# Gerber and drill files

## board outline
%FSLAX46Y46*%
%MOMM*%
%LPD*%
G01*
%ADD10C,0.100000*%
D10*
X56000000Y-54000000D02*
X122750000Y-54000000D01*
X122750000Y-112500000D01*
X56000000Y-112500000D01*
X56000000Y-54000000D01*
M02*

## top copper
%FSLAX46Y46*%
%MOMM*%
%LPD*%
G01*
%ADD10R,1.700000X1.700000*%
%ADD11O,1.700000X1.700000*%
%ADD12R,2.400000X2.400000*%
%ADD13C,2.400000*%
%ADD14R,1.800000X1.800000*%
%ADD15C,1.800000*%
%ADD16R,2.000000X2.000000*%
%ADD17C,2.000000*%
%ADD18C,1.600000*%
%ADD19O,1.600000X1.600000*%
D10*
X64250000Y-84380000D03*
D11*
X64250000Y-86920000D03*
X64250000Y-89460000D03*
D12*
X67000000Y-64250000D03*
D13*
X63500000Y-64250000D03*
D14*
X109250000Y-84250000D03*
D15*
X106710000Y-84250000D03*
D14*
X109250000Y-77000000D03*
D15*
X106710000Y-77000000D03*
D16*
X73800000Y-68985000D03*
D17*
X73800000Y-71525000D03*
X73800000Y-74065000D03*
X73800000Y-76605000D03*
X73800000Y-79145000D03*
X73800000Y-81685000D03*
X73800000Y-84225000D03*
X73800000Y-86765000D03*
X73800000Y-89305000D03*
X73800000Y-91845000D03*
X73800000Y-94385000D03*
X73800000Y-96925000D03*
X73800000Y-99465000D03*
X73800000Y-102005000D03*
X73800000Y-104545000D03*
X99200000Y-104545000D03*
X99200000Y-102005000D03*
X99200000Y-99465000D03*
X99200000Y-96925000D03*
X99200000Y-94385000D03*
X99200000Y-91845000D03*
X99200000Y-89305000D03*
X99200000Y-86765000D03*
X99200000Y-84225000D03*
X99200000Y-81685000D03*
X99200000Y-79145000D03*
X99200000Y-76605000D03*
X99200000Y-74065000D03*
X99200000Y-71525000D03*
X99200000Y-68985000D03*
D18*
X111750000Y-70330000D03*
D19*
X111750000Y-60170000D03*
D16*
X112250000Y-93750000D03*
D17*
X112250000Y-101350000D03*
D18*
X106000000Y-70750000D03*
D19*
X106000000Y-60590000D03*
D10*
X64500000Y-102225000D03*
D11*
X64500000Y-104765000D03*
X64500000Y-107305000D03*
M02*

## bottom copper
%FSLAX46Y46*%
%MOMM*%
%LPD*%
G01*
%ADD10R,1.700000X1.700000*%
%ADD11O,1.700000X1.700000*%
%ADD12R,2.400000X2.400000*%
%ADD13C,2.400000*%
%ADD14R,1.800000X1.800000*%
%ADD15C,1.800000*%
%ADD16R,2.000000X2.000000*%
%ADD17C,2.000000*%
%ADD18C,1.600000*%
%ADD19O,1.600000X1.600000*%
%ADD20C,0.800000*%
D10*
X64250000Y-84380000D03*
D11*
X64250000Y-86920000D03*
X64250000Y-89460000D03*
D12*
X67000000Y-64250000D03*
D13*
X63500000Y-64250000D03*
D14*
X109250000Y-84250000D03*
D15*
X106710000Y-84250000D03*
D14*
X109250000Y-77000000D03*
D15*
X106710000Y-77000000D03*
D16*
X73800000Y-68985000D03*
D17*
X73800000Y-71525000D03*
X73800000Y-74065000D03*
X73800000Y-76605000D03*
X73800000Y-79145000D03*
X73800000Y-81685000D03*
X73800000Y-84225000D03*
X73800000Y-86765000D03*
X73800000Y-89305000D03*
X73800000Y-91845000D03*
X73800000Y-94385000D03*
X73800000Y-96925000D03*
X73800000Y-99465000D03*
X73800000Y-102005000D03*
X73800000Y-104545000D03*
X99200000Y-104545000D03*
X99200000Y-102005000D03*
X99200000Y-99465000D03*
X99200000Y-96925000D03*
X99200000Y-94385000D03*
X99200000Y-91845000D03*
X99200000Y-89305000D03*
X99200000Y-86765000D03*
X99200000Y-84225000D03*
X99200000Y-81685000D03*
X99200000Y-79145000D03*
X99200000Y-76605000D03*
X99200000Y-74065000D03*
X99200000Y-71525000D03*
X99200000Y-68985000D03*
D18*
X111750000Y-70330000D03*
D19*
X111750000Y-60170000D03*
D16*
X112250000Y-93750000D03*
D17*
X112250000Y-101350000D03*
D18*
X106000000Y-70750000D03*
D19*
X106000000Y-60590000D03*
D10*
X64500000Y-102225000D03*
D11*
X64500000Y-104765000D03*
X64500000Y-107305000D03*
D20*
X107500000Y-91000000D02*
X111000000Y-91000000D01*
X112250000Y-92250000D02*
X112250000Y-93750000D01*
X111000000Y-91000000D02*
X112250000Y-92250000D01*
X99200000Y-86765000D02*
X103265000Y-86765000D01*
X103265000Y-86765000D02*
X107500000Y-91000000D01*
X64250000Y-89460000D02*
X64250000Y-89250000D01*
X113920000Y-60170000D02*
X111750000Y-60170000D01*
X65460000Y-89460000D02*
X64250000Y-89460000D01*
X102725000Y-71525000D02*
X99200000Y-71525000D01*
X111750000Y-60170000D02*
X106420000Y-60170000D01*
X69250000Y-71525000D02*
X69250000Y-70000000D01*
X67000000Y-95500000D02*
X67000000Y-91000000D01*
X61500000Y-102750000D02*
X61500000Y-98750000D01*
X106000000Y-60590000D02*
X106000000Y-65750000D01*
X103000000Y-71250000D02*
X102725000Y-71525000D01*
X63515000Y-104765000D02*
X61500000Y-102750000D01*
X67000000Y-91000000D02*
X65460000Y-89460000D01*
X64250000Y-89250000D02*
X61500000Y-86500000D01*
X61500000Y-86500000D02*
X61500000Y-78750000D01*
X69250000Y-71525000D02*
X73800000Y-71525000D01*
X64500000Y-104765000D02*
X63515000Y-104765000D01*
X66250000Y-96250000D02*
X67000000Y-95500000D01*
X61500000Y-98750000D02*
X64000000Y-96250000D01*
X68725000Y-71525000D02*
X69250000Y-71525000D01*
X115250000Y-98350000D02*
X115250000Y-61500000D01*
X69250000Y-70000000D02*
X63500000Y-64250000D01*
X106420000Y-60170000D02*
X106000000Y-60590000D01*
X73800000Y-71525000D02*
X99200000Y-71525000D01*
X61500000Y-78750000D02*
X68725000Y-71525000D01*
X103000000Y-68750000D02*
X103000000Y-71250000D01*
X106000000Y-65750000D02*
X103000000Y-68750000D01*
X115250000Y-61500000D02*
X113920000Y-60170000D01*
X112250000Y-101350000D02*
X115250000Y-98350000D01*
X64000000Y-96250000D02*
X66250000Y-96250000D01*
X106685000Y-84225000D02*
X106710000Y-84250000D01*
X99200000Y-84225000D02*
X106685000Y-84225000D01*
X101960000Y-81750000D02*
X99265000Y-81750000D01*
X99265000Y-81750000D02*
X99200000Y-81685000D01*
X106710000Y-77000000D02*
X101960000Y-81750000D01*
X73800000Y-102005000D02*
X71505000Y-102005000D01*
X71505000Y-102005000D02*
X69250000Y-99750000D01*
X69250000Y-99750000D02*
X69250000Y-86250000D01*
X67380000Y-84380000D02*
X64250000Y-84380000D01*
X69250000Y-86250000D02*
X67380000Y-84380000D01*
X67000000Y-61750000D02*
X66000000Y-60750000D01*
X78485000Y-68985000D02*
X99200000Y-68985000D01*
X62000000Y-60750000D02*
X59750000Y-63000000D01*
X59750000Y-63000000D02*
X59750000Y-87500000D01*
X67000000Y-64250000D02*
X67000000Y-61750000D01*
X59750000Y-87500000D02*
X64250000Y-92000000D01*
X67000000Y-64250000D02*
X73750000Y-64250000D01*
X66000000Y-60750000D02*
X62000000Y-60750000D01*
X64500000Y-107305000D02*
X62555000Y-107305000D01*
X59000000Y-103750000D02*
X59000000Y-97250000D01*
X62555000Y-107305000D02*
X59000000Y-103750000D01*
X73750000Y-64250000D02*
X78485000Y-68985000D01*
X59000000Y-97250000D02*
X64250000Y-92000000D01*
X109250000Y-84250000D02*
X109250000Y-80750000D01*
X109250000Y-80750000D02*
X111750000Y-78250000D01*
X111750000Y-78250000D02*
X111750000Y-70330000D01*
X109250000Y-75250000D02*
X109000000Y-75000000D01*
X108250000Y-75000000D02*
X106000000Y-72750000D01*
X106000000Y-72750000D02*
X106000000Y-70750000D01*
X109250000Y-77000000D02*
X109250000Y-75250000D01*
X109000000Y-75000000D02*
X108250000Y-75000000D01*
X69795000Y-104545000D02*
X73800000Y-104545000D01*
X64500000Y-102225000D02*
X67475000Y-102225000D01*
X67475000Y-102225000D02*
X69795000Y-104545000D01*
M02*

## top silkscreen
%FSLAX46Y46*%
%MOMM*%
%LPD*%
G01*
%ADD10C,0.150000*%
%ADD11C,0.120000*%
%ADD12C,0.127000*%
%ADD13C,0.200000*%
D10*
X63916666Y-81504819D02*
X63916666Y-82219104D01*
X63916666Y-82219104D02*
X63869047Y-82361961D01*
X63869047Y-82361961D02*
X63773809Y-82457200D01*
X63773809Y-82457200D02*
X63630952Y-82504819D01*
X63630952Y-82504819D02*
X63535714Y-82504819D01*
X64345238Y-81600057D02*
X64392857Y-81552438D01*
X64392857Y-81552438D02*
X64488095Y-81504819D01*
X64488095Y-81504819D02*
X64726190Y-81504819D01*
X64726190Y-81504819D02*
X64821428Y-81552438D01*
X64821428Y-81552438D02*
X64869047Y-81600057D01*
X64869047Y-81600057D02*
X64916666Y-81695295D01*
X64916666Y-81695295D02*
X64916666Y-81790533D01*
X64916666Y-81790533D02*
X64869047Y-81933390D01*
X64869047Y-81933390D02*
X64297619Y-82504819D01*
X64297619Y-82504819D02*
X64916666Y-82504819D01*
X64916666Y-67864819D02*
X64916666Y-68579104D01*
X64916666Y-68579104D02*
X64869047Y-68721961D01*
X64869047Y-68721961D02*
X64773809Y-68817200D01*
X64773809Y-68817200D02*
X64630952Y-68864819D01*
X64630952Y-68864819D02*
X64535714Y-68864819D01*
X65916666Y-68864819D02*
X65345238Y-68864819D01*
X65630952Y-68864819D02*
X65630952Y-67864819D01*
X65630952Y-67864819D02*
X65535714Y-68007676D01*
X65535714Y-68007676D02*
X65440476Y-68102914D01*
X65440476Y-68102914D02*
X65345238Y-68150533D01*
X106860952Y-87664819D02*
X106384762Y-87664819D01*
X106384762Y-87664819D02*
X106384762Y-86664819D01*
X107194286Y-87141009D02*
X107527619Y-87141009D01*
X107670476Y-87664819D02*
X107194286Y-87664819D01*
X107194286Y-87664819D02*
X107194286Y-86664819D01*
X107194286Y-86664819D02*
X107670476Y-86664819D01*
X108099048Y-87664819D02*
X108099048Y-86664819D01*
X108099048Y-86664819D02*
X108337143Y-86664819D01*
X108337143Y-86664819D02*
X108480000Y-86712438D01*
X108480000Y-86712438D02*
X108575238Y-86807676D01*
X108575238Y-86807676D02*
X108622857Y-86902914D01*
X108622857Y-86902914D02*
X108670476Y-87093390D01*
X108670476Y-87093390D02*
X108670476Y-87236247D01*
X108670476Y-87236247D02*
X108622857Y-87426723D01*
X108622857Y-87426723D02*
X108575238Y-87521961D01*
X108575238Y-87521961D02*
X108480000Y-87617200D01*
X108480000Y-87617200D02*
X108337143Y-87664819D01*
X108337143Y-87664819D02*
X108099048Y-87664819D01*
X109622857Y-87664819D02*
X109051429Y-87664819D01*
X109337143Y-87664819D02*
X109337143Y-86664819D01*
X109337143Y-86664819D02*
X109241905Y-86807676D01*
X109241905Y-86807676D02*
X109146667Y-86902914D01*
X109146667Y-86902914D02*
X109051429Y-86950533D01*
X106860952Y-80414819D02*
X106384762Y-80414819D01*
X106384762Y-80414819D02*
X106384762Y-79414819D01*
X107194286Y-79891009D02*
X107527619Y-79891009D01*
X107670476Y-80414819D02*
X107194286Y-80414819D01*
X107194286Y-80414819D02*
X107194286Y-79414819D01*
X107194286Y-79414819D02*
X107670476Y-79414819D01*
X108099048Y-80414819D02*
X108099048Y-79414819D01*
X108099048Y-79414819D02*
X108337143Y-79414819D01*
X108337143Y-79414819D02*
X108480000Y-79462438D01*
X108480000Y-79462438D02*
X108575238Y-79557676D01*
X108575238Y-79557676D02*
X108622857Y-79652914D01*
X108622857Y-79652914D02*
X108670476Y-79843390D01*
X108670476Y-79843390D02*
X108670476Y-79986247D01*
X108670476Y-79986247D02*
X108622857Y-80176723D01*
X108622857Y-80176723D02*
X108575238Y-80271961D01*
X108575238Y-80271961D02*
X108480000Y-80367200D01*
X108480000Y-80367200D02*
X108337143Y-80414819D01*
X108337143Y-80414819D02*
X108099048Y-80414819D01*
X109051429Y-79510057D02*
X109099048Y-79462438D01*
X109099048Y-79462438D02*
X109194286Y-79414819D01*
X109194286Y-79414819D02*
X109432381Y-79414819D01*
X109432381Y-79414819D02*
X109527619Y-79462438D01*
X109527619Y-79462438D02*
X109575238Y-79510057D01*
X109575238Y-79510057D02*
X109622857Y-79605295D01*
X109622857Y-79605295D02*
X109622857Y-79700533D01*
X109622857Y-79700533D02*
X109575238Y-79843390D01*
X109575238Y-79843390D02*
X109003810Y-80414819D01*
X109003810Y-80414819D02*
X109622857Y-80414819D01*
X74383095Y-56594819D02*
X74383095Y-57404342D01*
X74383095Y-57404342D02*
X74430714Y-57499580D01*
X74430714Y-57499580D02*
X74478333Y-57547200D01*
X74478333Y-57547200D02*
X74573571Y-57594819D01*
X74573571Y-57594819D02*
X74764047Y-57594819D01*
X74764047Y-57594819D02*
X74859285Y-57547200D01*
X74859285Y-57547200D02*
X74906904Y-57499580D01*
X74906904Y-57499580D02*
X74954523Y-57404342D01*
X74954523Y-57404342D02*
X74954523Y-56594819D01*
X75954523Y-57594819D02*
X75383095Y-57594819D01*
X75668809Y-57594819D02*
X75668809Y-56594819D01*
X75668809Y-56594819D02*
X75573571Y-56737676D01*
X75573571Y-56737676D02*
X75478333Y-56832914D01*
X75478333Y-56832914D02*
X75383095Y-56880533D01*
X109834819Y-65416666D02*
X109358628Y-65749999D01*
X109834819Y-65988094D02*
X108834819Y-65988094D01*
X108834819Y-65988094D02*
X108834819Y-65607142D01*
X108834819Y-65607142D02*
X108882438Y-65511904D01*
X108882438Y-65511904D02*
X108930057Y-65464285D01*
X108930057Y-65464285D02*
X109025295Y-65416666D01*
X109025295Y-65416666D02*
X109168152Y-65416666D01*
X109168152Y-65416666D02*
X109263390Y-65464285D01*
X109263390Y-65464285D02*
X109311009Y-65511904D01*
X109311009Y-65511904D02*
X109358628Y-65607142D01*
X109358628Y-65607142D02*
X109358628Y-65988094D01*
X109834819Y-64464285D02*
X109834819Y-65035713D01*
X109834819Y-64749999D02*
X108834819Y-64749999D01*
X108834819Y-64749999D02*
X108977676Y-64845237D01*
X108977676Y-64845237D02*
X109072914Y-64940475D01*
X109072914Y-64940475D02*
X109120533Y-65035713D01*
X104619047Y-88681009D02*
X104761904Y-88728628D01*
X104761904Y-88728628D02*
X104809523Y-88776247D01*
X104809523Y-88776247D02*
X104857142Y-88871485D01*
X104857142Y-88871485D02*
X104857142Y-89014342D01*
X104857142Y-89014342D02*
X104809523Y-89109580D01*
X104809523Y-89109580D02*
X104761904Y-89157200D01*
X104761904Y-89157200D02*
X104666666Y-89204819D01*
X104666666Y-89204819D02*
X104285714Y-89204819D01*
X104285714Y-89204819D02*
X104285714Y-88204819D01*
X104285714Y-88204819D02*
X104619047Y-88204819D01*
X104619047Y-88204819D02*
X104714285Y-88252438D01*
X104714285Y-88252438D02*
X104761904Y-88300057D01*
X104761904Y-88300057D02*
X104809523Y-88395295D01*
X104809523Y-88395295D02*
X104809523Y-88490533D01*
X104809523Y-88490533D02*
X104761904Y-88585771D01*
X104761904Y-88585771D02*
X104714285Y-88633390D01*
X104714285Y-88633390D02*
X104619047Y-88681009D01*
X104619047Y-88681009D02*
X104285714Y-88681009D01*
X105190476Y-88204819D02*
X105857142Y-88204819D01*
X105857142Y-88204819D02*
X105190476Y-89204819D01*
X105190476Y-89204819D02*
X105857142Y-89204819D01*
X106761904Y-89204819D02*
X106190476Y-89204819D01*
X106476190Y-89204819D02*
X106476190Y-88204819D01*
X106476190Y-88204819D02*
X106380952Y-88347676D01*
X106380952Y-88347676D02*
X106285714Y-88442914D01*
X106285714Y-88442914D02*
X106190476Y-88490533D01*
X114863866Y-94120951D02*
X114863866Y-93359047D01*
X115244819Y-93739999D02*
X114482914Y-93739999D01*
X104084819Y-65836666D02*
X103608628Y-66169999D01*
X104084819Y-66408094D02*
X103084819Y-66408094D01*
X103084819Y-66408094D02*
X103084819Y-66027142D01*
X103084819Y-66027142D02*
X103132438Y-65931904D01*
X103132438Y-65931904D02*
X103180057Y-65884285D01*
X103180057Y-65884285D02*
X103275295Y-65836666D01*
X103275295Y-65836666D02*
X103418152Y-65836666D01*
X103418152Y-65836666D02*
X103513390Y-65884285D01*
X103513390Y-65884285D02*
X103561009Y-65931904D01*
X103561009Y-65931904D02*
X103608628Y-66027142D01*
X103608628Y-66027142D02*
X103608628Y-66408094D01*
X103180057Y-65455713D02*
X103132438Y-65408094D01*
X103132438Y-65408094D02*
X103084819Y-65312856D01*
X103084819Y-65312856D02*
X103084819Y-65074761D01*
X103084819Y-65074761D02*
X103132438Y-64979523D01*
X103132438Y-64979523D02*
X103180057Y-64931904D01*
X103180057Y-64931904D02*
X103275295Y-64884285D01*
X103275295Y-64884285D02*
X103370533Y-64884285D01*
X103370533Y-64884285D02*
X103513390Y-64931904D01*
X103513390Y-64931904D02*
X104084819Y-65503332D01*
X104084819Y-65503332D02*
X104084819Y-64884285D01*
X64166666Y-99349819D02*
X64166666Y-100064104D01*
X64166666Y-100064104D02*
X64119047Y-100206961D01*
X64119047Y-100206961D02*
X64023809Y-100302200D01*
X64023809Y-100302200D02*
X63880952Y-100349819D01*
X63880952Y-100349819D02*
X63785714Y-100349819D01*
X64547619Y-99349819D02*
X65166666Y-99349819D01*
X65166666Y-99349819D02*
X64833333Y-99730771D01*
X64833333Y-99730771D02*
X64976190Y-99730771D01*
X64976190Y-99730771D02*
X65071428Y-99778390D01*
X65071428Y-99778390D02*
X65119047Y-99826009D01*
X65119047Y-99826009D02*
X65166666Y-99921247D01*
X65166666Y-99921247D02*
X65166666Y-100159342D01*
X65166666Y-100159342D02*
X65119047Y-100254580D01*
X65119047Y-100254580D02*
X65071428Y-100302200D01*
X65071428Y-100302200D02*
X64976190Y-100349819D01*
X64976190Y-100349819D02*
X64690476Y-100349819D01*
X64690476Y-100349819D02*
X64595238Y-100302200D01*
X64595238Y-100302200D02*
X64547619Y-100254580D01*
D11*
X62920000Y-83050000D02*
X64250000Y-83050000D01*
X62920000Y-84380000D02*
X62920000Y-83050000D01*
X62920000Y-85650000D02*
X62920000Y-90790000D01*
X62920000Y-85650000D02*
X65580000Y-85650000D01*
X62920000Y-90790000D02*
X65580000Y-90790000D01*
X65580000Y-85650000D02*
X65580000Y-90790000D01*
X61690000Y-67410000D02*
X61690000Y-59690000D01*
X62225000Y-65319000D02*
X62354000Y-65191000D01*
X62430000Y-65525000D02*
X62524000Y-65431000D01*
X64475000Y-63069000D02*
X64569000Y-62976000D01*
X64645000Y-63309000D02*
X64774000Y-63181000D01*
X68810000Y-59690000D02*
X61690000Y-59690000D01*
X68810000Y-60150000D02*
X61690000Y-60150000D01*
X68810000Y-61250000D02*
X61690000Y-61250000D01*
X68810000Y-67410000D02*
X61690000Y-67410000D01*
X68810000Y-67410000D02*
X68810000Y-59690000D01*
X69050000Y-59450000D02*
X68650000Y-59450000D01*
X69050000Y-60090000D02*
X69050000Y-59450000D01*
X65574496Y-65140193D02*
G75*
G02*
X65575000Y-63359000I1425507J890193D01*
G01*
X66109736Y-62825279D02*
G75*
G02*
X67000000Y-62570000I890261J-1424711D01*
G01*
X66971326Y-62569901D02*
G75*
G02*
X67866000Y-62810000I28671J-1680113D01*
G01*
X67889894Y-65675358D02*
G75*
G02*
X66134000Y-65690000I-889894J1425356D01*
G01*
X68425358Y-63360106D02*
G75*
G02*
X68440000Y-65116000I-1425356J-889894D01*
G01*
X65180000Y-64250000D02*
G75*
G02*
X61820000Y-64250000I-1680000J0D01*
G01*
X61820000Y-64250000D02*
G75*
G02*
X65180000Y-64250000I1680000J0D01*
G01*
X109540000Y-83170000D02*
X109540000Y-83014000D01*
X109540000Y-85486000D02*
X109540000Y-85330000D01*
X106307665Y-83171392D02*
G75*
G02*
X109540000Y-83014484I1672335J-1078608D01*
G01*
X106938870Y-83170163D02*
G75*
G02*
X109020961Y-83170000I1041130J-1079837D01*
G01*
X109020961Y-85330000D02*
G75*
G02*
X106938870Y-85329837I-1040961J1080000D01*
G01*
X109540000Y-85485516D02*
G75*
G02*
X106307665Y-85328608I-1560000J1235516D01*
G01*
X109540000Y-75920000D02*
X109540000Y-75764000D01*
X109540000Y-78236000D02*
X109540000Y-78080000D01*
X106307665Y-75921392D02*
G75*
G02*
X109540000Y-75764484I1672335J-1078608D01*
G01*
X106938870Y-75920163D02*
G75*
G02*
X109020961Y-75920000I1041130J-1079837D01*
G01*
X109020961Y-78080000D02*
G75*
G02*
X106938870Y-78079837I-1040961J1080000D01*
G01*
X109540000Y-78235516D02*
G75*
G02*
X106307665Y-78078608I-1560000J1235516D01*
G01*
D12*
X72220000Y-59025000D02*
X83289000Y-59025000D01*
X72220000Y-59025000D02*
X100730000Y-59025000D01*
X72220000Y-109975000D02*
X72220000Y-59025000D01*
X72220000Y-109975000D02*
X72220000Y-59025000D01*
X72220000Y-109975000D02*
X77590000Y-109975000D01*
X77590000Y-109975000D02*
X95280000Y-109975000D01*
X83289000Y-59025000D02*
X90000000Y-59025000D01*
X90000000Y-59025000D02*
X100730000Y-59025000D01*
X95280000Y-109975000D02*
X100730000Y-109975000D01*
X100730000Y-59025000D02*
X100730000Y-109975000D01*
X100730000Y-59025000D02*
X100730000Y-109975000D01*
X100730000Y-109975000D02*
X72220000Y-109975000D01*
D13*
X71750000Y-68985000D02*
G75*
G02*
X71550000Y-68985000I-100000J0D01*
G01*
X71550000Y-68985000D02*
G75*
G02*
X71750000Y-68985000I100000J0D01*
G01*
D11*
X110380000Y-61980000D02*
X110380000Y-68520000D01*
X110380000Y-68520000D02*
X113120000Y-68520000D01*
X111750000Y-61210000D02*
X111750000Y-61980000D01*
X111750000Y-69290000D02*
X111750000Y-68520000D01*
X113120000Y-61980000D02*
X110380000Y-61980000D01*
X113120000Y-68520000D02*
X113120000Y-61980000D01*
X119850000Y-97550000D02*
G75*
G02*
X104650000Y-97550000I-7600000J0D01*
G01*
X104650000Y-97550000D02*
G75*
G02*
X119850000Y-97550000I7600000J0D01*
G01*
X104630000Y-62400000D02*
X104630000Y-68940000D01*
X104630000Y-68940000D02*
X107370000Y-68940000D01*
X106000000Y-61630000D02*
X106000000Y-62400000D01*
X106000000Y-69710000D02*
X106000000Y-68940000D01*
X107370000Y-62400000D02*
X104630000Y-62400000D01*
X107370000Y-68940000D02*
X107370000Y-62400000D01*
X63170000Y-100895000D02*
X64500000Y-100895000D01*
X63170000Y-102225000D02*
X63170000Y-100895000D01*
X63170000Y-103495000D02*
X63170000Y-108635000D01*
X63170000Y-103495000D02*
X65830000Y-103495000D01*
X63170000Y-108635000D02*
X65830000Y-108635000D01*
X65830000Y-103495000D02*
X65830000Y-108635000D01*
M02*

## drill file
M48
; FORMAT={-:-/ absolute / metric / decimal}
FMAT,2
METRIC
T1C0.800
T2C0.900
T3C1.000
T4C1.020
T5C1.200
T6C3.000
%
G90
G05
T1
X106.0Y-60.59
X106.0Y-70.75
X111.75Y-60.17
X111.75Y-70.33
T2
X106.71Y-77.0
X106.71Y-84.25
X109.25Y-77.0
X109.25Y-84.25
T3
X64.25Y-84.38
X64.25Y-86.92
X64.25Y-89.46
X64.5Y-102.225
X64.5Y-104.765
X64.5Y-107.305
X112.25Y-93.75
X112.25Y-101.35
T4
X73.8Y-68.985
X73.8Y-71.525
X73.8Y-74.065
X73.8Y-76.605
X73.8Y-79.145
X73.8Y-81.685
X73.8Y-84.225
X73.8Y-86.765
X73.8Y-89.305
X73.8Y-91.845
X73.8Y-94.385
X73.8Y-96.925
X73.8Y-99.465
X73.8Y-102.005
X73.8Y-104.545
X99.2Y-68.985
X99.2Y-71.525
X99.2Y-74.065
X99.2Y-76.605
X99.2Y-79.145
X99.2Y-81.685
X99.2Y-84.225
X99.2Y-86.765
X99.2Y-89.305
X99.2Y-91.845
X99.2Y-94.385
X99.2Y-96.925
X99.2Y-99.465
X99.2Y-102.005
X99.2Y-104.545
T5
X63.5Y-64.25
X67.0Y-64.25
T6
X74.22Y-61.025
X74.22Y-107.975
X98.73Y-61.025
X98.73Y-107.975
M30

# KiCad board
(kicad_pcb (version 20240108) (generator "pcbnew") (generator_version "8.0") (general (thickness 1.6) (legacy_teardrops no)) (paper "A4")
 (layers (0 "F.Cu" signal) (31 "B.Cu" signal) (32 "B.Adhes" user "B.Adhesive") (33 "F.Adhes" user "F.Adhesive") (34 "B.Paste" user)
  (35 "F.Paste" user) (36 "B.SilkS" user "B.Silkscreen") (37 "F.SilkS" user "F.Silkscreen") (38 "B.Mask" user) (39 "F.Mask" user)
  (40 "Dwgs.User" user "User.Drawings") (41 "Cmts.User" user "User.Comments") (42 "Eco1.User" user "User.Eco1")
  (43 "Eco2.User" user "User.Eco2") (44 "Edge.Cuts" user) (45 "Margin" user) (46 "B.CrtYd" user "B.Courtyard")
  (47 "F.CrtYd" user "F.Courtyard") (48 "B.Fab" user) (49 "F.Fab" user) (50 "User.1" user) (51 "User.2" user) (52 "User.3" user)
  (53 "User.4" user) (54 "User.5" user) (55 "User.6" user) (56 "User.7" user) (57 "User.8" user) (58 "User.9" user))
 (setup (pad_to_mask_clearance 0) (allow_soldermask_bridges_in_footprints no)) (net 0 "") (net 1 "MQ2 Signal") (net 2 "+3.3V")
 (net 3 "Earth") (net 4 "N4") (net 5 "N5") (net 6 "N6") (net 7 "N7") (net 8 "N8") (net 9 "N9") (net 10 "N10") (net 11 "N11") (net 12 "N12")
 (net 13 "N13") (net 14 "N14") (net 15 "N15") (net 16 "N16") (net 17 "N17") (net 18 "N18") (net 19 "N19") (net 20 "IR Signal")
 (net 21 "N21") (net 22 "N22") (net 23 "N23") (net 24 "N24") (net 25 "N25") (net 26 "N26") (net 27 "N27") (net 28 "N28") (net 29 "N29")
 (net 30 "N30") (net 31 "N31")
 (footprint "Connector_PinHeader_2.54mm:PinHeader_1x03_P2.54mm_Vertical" (layer "F.Cu") (at 64.25 84.38)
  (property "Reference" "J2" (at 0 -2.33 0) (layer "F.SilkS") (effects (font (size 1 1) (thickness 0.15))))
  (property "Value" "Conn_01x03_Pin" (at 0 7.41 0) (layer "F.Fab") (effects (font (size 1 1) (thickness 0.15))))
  (fp_line (start -1.33 -1.33) (end 0 -1.33) (stroke (width 0.12) (type solid)) (layer "F.SilkS"))
  (fp_line (start -1.33 0) (end -1.33 -1.33) (stroke (width 0.12) (type solid)) (layer "F.SilkS"))
  (fp_line (start -1.33 1.27) (end -1.33 6.41) (stroke (width 0.12) (type solid)) (layer "F.SilkS"))
  (fp_line (start -1.33 1.27) (end 1.33 1.27) (stroke (width 0.12) (type solid)) (layer "F.SilkS"))
  (fp_line (start -1.33 6.41) (end 1.33 6.41) (stroke (width 0.12) (type solid)) (layer "F.SilkS"))
  (fp_line (start 1.33 1.27) (end 1.33 6.41) (stroke (width 0.12) (type solid)) (layer "F.SilkS"))
  (pad "1" thru_hole rect (at 0 0) (size 1.7 1.7) (drill 1) (layers "*.Cu" "*.Mask") (remove_unused_layers no) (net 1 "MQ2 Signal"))
  (pad "2" thru_hole oval (at 0 2.54) (size 1.7 1.7) (drill 1) (layers "*.Cu" "*.Mask") (remove_unused_layers no) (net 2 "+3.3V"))
  (pad "3" thru_hole oval (at 0 5.08) (size 1.7 1.7) (drill 1) (layers "*.Cu" "*.Mask") (remove_unused_layers no) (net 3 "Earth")))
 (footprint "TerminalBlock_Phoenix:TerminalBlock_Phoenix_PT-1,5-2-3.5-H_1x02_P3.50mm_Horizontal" (layer "F.Cu") (at 67 64.25 180)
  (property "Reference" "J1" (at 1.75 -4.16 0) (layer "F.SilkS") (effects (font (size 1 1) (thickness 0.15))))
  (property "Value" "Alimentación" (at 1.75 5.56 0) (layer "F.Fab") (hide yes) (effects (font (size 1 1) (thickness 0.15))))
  (fp_line (start 5.31 -3.16) (end 5.31 4.56) (stroke (width 0.12) (type solid)) (layer "F.SilkS"))
  (fp_line (start 4.775 -1.069) (end 4.646 -0.941) (stroke (width 0.12) (type solid)) (layer "F.SilkS"))
  (fp_line (start 4.57 -1.275) (end 4.476 -1.181) (stroke (width 0.12) (type solid)) (layer "F.SilkS"))
  (fp_line (start 2.525 1.181) (end 2.431 1.274) (stroke (width 0.12) (type solid)) (layer "F.SilkS"))
  (fp_line (start 2.355 0.941) (end 2.226 1.069) (stroke (width 0.12) (type solid)) (layer "F.SilkS"))
  (fp_line (start -1.81 4.56) (end 5.31 4.56) (stroke (width 0.12) (type solid)) (layer "F.SilkS"))
  (fp_line (start -1.81 4.1) (end 5.31 4.1) (stroke (width 0.12) (type solid)) (layer "F.SilkS"))
  (fp_line (start -1.81 3) (end 5.31 3) (stroke (width 0.12) (type solid)) (layer "F.SilkS"))
  (fp_line (start -1.81 -3.16) (end 5.31 -3.16) (stroke (width 0.12) (type solid)) (layer "F.SilkS"))
  (fp_line (start -1.81 -3.16) (end -1.81 4.56) (stroke (width 0.12) (type solid)) (layer "F.SilkS"))
  (fp_line (start -2.05 4.8) (end -1.65 4.8) (stroke (width 0.12) (type solid)) (layer "F.SilkS"))
  (fp_line (start -2.05 4.16) (end -2.05 4.8) (stroke (width 0.12) (type solid)) (layer "F.SilkS"))
  (fp_arc (start 1.425504 -0.890193) (mid 1.680626 0.000476) (end 1.425 0.891) (stroke (width 0.12) (type solid)) (layer "F.SilkS"))
  (fp_arc (start 0.890264 1.424721) (mid 0.463071 1.61492) (end 0 1.68) (stroke (width 0.12) (type solid)) (layer "F.SilkS"))
  (fp_arc (start 0.028674 1.680099) (mid -0.435535 1.622918) (end -0.866 1.44) (stroke (width 0.12) (type solid)) (layer "F.SilkS"))
  (fp_arc (start -0.889894 -1.425358) (mid -0.014012 -1.680286) (end 0.866 -1.44) (stroke (width 0.12) (type solid)) (layer "F.SilkS"))
  (fp_arc (start -1.425358 0.889894) (mid -1.680286 0.014012) (end -1.44 -0.866) (stroke (width 0.12) (type solid)) (layer "F.SilkS"))
  (fp_circle (center 3.5 0) (end 5.18 0) (stroke (width 0.12) (type solid)) (fill none) (layer "F.SilkS"))
  (pad "1" thru_hole rect (at 0 0 180) (size 2.4 2.4) (drill 1.2) (layers "*.Cu" "*.Mask") (remove_unused_layers no) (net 2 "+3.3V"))
  (pad "2" thru_hole circle (at 3.5 0 180) (size 2.4 2.4) (drill 1.2) (layers "*.Cu" "*.Mask") (remove_unused_layers no) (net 3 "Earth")))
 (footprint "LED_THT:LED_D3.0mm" (layer "F.Cu") (at 109.25 84.25 180)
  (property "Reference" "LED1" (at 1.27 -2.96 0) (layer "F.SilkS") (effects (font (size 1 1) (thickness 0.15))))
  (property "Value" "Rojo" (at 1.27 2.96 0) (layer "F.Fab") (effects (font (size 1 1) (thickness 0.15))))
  (fp_line (start -0.29 1.08) (end -0.29 1.236) (stroke (width 0.12) (type solid)) (layer "F.SilkS"))
  (fp_line (start -0.29 -1.236) (end -0.29 -1.08) (stroke (width 0.12) (type solid)) (layer "F.SilkS"))
  (fp_arc (start 2.942335 1.078608) (mid 1.366487 1.987659) (end -0.29 1.235516) (stroke (width 0.12) (type solid)) (layer "F.SilkS"))
  (fp_arc (start 2.31113 1.079837) (mid 1.270117 1.5) (end 0.229039 1.08) (stroke (width 0.12) (type solid)) (layer "F.SilkS"))
  (fp_arc (start 0.229039 -1.08) (mid 1.270117 -1.5) (end 2.31113 -1.079837) (stroke (width 0.12) (type solid)) (layer "F.SilkS"))
  (fp_arc (start -0.29 -1.235516) (mid 1.366487 -1.987659) (end 2.942335 -1.078608) (stroke (width 0.12) (type solid)) (layer "F.SilkS"))
  (pad "1" thru_hole rect (at 0 0 180) (size 1.8 1.8) (drill 0.9) (layers "*.Cu" "*.Mask") (remove_unused_layers no) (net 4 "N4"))
  (pad "2" thru_hole circle (at 2.54 0 180) (size 1.8 1.8) (drill 0.9) (layers "*.Cu" "*.Mask") (remove_unused_layers no) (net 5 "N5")))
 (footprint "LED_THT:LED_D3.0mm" (layer "F.Cu") (at 109.25 77 180)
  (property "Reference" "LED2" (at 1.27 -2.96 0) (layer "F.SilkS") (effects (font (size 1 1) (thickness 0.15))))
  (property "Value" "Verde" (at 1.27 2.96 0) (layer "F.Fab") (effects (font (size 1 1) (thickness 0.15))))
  (fp_line (start -0.29 1.08) (end -0.29 1.236) (stroke (width 0.12) (type solid)) (layer "F.SilkS"))
  (fp_line (start -0.29 -1.236) (end -0.29 -1.08) (stroke (width 0.12) (type solid)) (layer "F.SilkS"))
  (fp_arc (start 2.942335 1.078608) (mid 1.366487 1.987659) (end -0.29 1.235516) (stroke (width 0.12) (type solid)) (layer "F.SilkS"))
  (fp_arc (start 2.31113 1.079837) (mid 1.270117 1.5) (end 0.229039 1.08) (stroke (width 0.12) (type solid)) (layer "F.SilkS"))
  (fp_arc (start 0.229039 -1.08) (mid 1.270117 -1.5) (end 2.31113 -1.079837) (stroke (width 0.12) (type solid)) (layer "F.SilkS"))
  (fp_arc (start -0.29 -1.235516) (mid 1.366487 -1.987659) (end 2.942335 -1.078608) (stroke (width 0.12) (type solid)) (layer "F.SilkS"))
  (pad "1" thru_hole rect (at 0 0 180) (size 1.8 1.8) (drill 0.9) (layers "*.Cu" "*.Mask") (remove_unused_layers no) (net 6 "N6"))
  (pad "2" thru_hole circle (at 2.54 0 180) (size 1.8 1.8) (drill 0.9) (layers "*.Cu" "*.Mask") (remove_unused_layers no) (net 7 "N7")))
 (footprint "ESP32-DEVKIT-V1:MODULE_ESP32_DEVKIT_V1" (layer "F.Cu") (at 86.5 84.5)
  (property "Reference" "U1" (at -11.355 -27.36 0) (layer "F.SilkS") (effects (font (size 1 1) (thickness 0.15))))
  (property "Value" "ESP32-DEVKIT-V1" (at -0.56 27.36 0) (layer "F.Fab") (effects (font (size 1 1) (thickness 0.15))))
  (fp_line (start -14.28 -25.475) (end -3.211 -25.475) (stroke (width 0.127) (type solid)) (layer "F.SilkS"))
  (fp_line (start -14.28 -25.475) (end 14.23 -25.475) (stroke (width 0.127) (type solid)) (layer "F.SilkS"))
  (fp_line (start -14.28 25.475) (end -14.28 -25.475) (stroke (width 0.127) (type solid)) (layer "F.SilkS"))
  (fp_line (start -14.28 25.475) (end -14.28 -25.475) (stroke (width 0.127) (type solid)) (layer "F.SilkS"))
  (fp_line (start -14.28 25.475) (end -8.91 25.475) (stroke (width 0.127) (type solid)) (layer "F.SilkS"))
  (fp_line (start -8.91 25.475) (end 8.78 25.475) (stroke (width 0.127) (type solid)) (layer "F.SilkS"))
  (fp_line (start -3.211 -25.475) (end 3.5 -25.475) (stroke (width 0.127) (type solid)) (layer "F.SilkS"))
  (fp_line (start 3.5 -25.475) (end 14.23 -25.475) (stroke (width 0.127) (type solid)) (layer "F.SilkS"))
  (fp_line (start 8.78 25.475) (end 14.23 25.475) (stroke (width 0.127) (type solid)) (layer "F.SilkS"))
  (fp_line (start 14.23 -25.475) (end 14.23 25.475) (stroke (width 0.127) (type solid)) (layer "F.SilkS"))
  (fp_line (start 14.23 -25.475) (end 14.23 25.475) (stroke (width 0.127) (type solid)) (layer "F.SilkS"))
  (fp_line (start 14.23 25.475) (end -14.28 25.475) (stroke (width 0.127) (type solid)) (layer "F.SilkS"))
  (fp_circle (center -14.85 -15.515) (end -14.75 -15.515) (stroke (width 0.2) (type solid)) (fill none) (layer "F.SilkS"))
  (pad "" np_thru_hole circle (at -12.28 -23.475) (size 3 3) (drill 3) (layers "*.Cu" "*.Mask"))
  (pad "" np_thru_hole circle (at -12.28 23.475) (size 3 3) (drill 3) (layers "*.Cu" "*.Mask"))
  (pad "" np_thru_hole circle (at 12.23 -23.475) (size 3 3) (drill 3) (layers "*.Cu" "*.Mask"))
  (pad "" np_thru_hole circle (at 12.23 23.475) (size 3 3) (drill 3) (layers "*.Cu" "*.Mask"))
  (pad "1" thru_hole rect (at -12.7 -15.515) (size 2 2) (drill 1.02) (layers "*.Cu" "*.Mask") (remove_unused_layers no) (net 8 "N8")
   (solder_mask_margin 0.102))
  (pad "2" thru_hole circle (at -12.7 -12.975) (size 2 2) (drill 1.02) (layers "*.Cu" "*.Mask") (remove_unused_layers no) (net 3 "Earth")
   (solder_mask_margin 0.102))
  (pad "3" thru_hole circle (at -12.7 -10.435) (size 2 2) (drill 1.02) (layers "*.Cu" "*.Mask") (remove_unused_layers no) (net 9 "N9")
   (solder_mask_margin 0.102))
  (pad "4" thru_hole circle (at -12.7 -7.895) (size 2 2) (drill 1.02) (layers "*.Cu" "*.Mask") (remove_unused_layers no) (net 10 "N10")
   (solder_mask_margin 0.102))
  (pad "5" thru_hole circle (at -12.7 -5.355) (size 2 2) (drill 1.02) (layers "*.Cu" "*.Mask") (remove_unused_layers no) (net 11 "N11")
   (solder_mask_margin 0.102))
  (pad "6" thru_hole circle (at -12.7 -2.815) (size 2 2) (drill 1.02) (layers "*.Cu" "*.Mask") (remove_unused_layers no) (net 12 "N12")
   (solder_mask_margin 0.102))
  (pad "7" thru_hole circle (at -12.7 -0.275) (size 2 2) (drill 1.02) (layers "*.Cu" "*.Mask") (remove_unused_layers no) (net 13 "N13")
   (solder_mask_margin 0.102))
  (pad "8" thru_hole circle (at -12.7 2.265) (size 2 2) (drill 1.02) (layers "*.Cu" "*.Mask") (remove_unused_layers no) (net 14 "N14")
   (solder_mask_margin 0.102))
  (pad "9" thru_hole circle (at -12.7 4.805) (size 2 2) (drill 1.02) (layers "*.Cu" "*.Mask") (remove_unused_layers no) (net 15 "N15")
   (solder_mask_margin 0.102))
  (pad "10" thru_hole circle (at -12.7 7.345) (size 2 2) (drill 1.02) (layers "*.Cu" "*.Mask") (remove_unused_layers no) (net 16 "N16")
   (solder_mask_margin 0.102))
  (pad "11" thru_hole circle (at -12.7 9.885) (size 2 2) (drill 1.02) (layers "*.Cu" "*.Mask") (remove_unused_layers no) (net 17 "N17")
   (solder_mask_margin 0.102))
  (pad "12" thru_hole circle (at -12.7 12.425) (size 2 2) (drill 1.02) (layers "*.Cu" "*.Mask") (remove_unused_layers no) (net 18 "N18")
   (solder_mask_margin 0.102))
  (pad "13" thru_hole circle (at -12.7 14.965) (size 2 2) (drill 1.02) (layers "*.Cu" "*.Mask") (remove_unused_layers no) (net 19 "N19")
   (solder_mask_margin 0.102))
  (pad "14" thru_hole circle (at -12.7 17.505) (size 2 2) (drill 1.02) (layers "*.Cu" "*.Mask") (remove_unused_layers no)
   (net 1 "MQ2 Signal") (solder_mask_margin 0.102))
  (pad "15" thru_hole circle (at -12.7 20.045) (size 2 2) (drill 1.02) (layers "*.Cu" "*.Mask") (remove_unused_layers no)
   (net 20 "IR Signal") (solder_mask_margin 0.102))
  (pad "16" thru_hole circle (at 12.7 20.045) (size 2 2) (drill 1.02) (layers "*.Cu" "*.Mask") (remove_unused_layers no) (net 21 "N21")
   (solder_mask_margin 0.102))
  (pad "17" thru_hole circle (at 12.7 17.505) (size 2 2) (drill 1.02) (layers "*.Cu" "*.Mask") (remove_unused_layers no) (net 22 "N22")
   (solder_mask_margin 0.102))
  (pad "18" thru_hole circle (at 12.7 14.965) (size 2 2) (drill 1.02) (layers "*.Cu" "*.Mask") (remove_unused_layers no) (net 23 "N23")
   (solder_mask_margin 0.102))
  (pad "19" thru_hole circle (at 12.7 12.425) (size 2 2) (drill 1.02) (layers "*.Cu" "*.Mask") (remove_unused_layers no) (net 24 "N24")
   (solder_mask_margin 0.102))
  (pad "20" thru_hole circle (at 12.7 9.885) (size 2 2) (drill 1.02) (layers "*.Cu" "*.Mask") (remove_unused_layers no) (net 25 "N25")
   (solder_mask_margin 0.102))
  (pad "21" thru_hole circle (at 12.7 7.345) (size 2 2) (drill 1.02) (layers "*.Cu" "*.Mask") (remove_unused_layers no) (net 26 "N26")
   (solder_mask_margin 0.102))
  (pad "22" thru_hole circle (at 12.7 4.805) (size 2 2) (drill 1.02) (layers "*.Cu" "*.Mask") (remove_unused_layers no) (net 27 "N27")
   (solder_mask_margin 0.102))
  (pad "23" thru_hole circle (at 12.7 2.265) (size 2 2) (drill 1.02) (layers "*.Cu" "*.Mask") (remove_unused_layers no) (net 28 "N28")
   (solder_mask_margin 0.102))
  (pad "24" thru_hole circle (at 12.7 -0.275) (size 2 2) (drill 1.02) (layers "*.Cu" "*.Mask") (remove_unused_layers no) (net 5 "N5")
   (solder_mask_margin 0.102))
  (pad "25" thru_hole circle (at 12.7 -2.815) (size 2 2) (drill 1.02) (layers "*.Cu" "*.Mask") (remove_unused_layers no) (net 7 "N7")
   (solder_mask_margin 0.102))
  (pad "26" thru_hole circle (at 12.7 -5.355) (size 2 2) (drill 1.02) (layers "*.Cu" "*.Mask") (remove_unused_layers no) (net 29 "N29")
   (solder_mask_margin 0.102))
  (pad "27" thru_hole circle (at 12.7 -7.895) (size 2 2) (drill 1.02) (layers "*.Cu" "*.Mask") (remove_unused_layers no) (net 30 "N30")
   (solder_mask_margin 0.102))
  (pad "28" thru_hole circle (at 12.7 -10.435) (size 2 2) (drill 1.02) (layers "*.Cu" "*.Mask") (remove_unused_layers no) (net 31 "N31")
   (solder_mask_margin 0.102))
  (pad "29" thru_hole circle (at 12.7 -12.975) (size 2 2) (drill 1.02) (layers "*.Cu" "*.Mask") (remove_unused_layers no) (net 3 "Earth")
   (solder_mask_margin 0.102))
  (pad "30" thru_hole circle (at 12.7 -15.515) (size 2 2) (drill 1.02) (layers "*.Cu" "*.Mask") (remove_unused_layers no) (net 2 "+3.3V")
   (solder_mask_margin 0.102))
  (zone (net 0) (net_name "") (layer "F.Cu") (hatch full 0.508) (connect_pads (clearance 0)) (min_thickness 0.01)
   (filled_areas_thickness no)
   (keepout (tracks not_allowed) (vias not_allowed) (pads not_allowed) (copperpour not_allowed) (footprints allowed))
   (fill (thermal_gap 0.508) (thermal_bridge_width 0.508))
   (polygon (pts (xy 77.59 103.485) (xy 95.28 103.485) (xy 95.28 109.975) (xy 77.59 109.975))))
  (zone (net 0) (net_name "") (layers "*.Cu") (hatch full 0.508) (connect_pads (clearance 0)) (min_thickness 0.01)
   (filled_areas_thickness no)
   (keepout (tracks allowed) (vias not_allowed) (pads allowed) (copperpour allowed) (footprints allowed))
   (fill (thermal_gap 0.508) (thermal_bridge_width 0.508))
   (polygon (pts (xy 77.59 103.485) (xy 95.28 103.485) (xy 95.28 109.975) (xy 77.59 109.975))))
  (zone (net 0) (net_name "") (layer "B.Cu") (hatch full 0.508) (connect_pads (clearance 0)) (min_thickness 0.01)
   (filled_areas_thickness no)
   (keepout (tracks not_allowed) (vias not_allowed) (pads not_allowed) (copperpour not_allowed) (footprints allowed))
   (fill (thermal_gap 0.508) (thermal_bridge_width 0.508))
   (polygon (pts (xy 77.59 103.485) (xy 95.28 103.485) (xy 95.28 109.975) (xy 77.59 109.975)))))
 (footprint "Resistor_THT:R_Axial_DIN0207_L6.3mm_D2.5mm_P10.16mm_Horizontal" (layer "F.Cu") (at 111.75 70.33 90)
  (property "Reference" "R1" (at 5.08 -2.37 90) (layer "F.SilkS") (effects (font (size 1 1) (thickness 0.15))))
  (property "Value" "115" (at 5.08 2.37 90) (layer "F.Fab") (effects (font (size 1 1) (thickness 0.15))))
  (fp_line (start 8.35 -1.37) (end 1.81 -1.37) (stroke (width 0.12) (type solid)) (layer "F.SilkS"))
  (fp_line (start 1.81 -1.37) (end 1.81 1.37) (stroke (width 0.12) (type solid)) (layer "F.SilkS"))
  (fp_line (start 9.12 0) (end 8.35 0) (stroke (width 0.12) (type solid)) (layer "F.SilkS"))
  (fp_line (start 1.04 0) (end 1.81 0) (stroke (width 0.12) (type solid)) (layer "F.SilkS"))
  (fp_line (start 8.35 1.37) (end 8.35 -1.37) (stroke (width 0.12) (type solid)) (layer "F.SilkS"))
  (fp_line (start 1.81 1.37) (end 8.35 1.37) (stroke (width 0.12) (type solid)) (layer "F.SilkS"))
  (pad "1" thru_hole circle (at 0 0 90) (size 1.6 1.6) (drill 0.8) (layers "*.Cu" "*.Mask") (remove_unused_layers no) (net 4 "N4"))
  (pad "2" thru_hole oval (at 10.16 0 90) (size 1.6 1.6) (drill 0.8) (layers "*.Cu" "*.Mask") (remove_unused_layers no) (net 3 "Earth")))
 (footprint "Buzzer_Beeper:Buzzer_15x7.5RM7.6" (layer "F.Cu") (at 112.25 93.75 -90)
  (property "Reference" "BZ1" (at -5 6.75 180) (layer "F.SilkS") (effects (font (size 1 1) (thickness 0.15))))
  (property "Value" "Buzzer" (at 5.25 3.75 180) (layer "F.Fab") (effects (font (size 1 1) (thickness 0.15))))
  (fp_circle (center 3.8 0) (end 11.4 0) (stroke (width 0.12) (type solid)) (fill none) (layer "F.SilkS"))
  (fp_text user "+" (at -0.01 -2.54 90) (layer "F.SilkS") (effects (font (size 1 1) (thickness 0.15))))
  (pad "1" thru_hole rect (at 0 0 270) (size 2 2) (drill 1) (layers "*.Cu" "*.Mask") (remove_unused_layers no) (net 28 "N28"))
  (pad "2" thru_hole circle (at 7.6 0 270) (size 2 2) (drill 1) (layers "*.Cu" "*.Mask") (remove_unused_layers no) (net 3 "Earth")))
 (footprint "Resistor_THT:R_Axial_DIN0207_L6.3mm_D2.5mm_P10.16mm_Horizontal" (layer "F.Cu") (at 106 70.75 90)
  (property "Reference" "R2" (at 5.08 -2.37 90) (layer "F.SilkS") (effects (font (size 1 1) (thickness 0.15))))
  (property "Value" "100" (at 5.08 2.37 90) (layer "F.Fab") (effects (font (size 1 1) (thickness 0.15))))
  (fp_line (start 8.35 -1.37) (end 1.81 -1.37) (stroke (width 0.12) (type solid)) (layer "F.SilkS"))
  (fp_line (start 1.81 -1.37) (end 1.81 1.37) (stroke (width 0.12) (type solid)) (layer "F.SilkS"))
  (fp_line (start 9.12 0) (end 8.35 0) (stroke (width 0.12) (type solid)) (layer "F.SilkS"))
  (fp_line (start 1.04 0) (end 1.81 0) (stroke (width 0.12) (type solid)) (layer "F.SilkS"))
  (fp_line (start 8.35 1.37) (end 8.35 -1.37) (stroke (width 0.12) (type solid)) (layer "F.SilkS"))
  (fp_line (start 1.81 1.37) (end 8.35 1.37) (stroke (width 0.12) (type solid)) (layer "F.SilkS"))
  (pad "1" thru_hole circle (at 0 0 90) (size 1.6 1.6) (drill 0.8) (layers "*.Cu" "*.Mask") (remove_unused_layers no) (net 6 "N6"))
  (pad "2" thru_hole oval (at 10.16 0 90) (size 1.6 1.6) (drill 0.8) (layers "*.Cu" "*.Mask") (remove_unused_layers no) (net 3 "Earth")))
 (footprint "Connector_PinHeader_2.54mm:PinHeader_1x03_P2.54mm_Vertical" (layer "F.Cu") (at 64.5 102.225)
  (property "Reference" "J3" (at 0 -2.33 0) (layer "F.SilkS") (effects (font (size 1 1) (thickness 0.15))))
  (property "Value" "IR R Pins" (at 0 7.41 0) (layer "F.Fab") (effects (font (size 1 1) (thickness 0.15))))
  (fp_line (start -1.33 -1.33) (end 0 -1.33) (stroke (width 0.12) (type solid)) (layer "F.SilkS"))
  (fp_line (start -1.33 0) (end -1.33 -1.33) (stroke (width 0.12) (type solid)) (layer "F.SilkS"))
  (fp_line (start -1.33 1.27) (end -1.33 6.41) (stroke (width 0.12) (type solid)) (layer "F.SilkS"))
  (fp_line (start -1.33 1.27) (end 1.33 1.27) (stroke (width 0.12) (type solid)) (layer "F.SilkS"))
  (fp_line (start -1.33 6.41) (end 1.33 6.41) (stroke (width 0.12) (type solid)) (layer "F.SilkS"))
  (fp_line (start 1.33 1.27) (end 1.33 6.41) (stroke (width 0.12) (type solid)) (layer "F.SilkS"))
  (pad "1" thru_hole rect (at 0 0) (size 1.7 1.7) (drill 1) (layers "*.Cu" "*.Mask") (remove_unused_layers no) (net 20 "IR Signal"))
  (pad "2" thru_hole oval (at 0 2.54) (size 1.7 1.7) (drill 1) (layers "*.Cu" "*.Mask") (remove_unused_layers no) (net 3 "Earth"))
  (pad "3" thru_hole oval (at 0 5.08) (size 1.7 1.7) (drill 1) (layers "*.Cu" "*.Mask") (remove_unused_layers no) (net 2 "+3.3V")))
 (gr_rect (start 56 54) (end 122.75 112.5) (stroke (width 0.1) (type default)) (fill none) (layer "Edge.Cuts"))
 (segment (start 107.5 91) (end 111 91) (width 0.8) (layer "B.Cu") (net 28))
 (segment (start 112.25 92.25) (end 112.25 93.75) (width 0.8) (layer "B.Cu") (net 28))
 (segment (start 111 91) (end 112.25 92.25) (width 0.8) (layer "B.Cu") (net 28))
 (segment (start 99.2 86.765) (end 103.265 86.765) (width 0.8) (layer "B.Cu") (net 28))
 (segment (start 103.265 86.765) (end 107.5 91) (width 0.8) (layer "B.Cu") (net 28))
 (segment (start 64.25 89.46) (end 64.25 89.25) (width 0.8) (layer "B.Cu") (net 3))
 (segment (start 113.92 60.17) (end 111.75 60.17) (width 0.8) (layer "B.Cu") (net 3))
 (segment (start 65.46 89.46) (end 64.25 89.46) (width 0.8) (layer "B.Cu") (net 3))
 (segment (start 102.725 71.525) (end 99.2 71.525) (width 0.8) (layer "B.Cu") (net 3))
 (segment (start 111.75 60.17) (end 106.42 60.17) (width 0.8) (layer "B.Cu") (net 3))
 (segment (start 69.25 71.525) (end 69.25 70) (width 0.8) (layer "B.Cu") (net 3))
 (segment (start 67 95.5) (end 67 91) (width 0.8) (layer "B.Cu") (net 3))
 (segment (start 61.5 102.75) (end 61.5 98.75) (width 0.8) (layer "B.Cu") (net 3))
 (segment (start 106 60.59) (end 106 65.75) (width 0.8) (layer "B.Cu") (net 3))
 (segment (start 103 71.25) (end 102.725 71.525) (width 0.8) (layer "B.Cu") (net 3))
 (segment (start 63.515 104.765) (end 61.5 102.75) (width 0.8) (layer "B.Cu") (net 3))
 (segment (start 67 91) (end 65.46 89.46) (width 0.8) (layer "B.Cu") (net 3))
 (segment (start 64.25 89.25) (end 61.5 86.5) (width 0.8) (layer "B.Cu") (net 3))
 (segment (start 61.5 86.5) (end 61.5 78.75) (width 0.8) (layer "B.Cu") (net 3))
 (segment (start 69.25 71.525) (end 73.8 71.525) (width 0.8) (layer "B.Cu") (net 3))
 (segment (start 64.5 104.765) (end 63.515 104.765) (width 0.8) (layer "B.Cu") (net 3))
 (segment (start 66.25 96.25) (end 67 95.5) (width 0.8) (layer "B.Cu") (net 3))
 (segment (start 61.5 98.75) (end 64 96.25) (width 0.8) (layer "B.Cu") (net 3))
 (segment (start 68.725 71.525) (end 69.25 71.525) (width 0.8) (layer "B.Cu") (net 3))
 (segment (start 115.25 98.35) (end 115.25 61.5) (width 0.8) (layer "B.Cu") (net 3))
 (segment (start 69.25 70) (end 63.5 64.25) (width 0.8) (layer "B.Cu") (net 3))
 (segment (start 106.42 60.17) (end 106 60.59) (width 0.8) (layer "B.Cu") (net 3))
 (segment (start 73.8 71.525) (end 99.2 71.525) (width 0.8) (layer "B.Cu") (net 3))
 (segment (start 61.5 78.75) (end 68.725 71.525) (width 0.8) (layer "B.Cu") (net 3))
 (segment (start 103 68.75) (end 103 71.25) (width 0.8) (layer "B.Cu") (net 3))
 (segment (start 106 65.75) (end 103 68.75) (width 0.8) (layer "B.Cu") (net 3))
 (segment (start 115.25 61.5) (end 113.92 60.17) (width 0.8) (layer "B.Cu") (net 3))
 (segment (start 112.25 101.35) (end 115.25 98.35) (width 0.8) (layer "B.Cu") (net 3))
 (segment (start 64 96.25) (end 66.25 96.25) (width 0.8) (layer "B.Cu") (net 3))
 (segment (start 106.685 84.225) (end 106.71 84.25) (width 0.8) (layer "B.Cu") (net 5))
 (segment (start 99.2 84.225) (end 106.685 84.225) (width 0.8) (layer "B.Cu") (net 5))
 (segment (start 101.96 81.75) (end 99.265 81.75) (width 0.8) (layer "B.Cu") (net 7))
 (segment (start 99.265 81.75) (end 99.2 81.685) (width 0.8) (layer "B.Cu") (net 7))
 (segment (start 106.71 77) (end 101.96 81.75) (width 0.8) (layer "B.Cu") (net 7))
 (segment (start 73.8 102.005) (end 71.505 102.005) (width 0.8) (layer "B.Cu") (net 1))
 (segment (start 71.505 102.005) (end 69.25 99.75) (width 0.8) (layer "B.Cu") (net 1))
 (segment (start 69.25 99.75) (end 69.25 86.25) (width 0.8) (layer "B.Cu") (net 1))
 (segment (start 67.38 84.38) (end 64.25 84.38) (width 0.8) (layer "B.Cu") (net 1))
 (segment (start 69.25 86.25) (end 67.38 84.38) (width 0.8) (layer "B.Cu") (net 1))
 (segment (start 67 61.75) (end 66 60.75) (width 0.8) (layer "B.Cu") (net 2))
 (segment (start 78.485 68.985) (end 99.2 68.985) (width 0.8) (layer "B.Cu") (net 2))
 (segment (start 62 60.75) (end 59.75 63) (width 0.8) (layer "B.Cu") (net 2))
 (segment (start 59.75 63) (end 59.75 87.5) (width 0.8) (layer "B.Cu") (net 2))
 (segment (start 67 64.25) (end 67 61.75) (width 0.8) (layer "B.Cu") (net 2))
 (segment (start 59.75 87.5) (end 64.25 92) (width 0.8) (layer "B.Cu") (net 2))
 (segment (start 67 64.25) (end 73.75 64.25) (width 0.8) (layer "B.Cu") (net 2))
 (segment (start 66 60.75) (end 62 60.75) (width 0.8) (layer "B.Cu") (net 2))
 (segment (start 64.5 107.305) (end 62.555 107.305) (width 0.8) (layer "B.Cu") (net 2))
 (segment (start 59 103.75) (end 59 97.25) (width 0.8) (layer "B.Cu") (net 2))
 (segment (start 62.555 107.305) (end 59 103.75) (width 0.8) (layer "B.Cu") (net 2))
 (segment (start 73.75 64.25) (end 78.485 68.985) (width 0.8) (layer "B.Cu") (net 2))
 (segment (start 59 97.25) (end 64.25 92) (width 0.8) (layer "B.Cu") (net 2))
 (segment (start 109.25 84.25) (end 109.25 80.75) (width 0.8) (layer "B.Cu") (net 4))
 (segment (start 109.25 80.75) (end 111.75 78.25) (width 0.8) (layer "B.Cu") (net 4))
 (segment (start 111.75 78.25) (end 111.75 70.33) (width 0.8) (layer "B.Cu") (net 4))
 (segment (start 109.25 75.25) (end 109 75) (width 0.8) (layer "B.Cu") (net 6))
 (segment (start 108.25 75) (end 106 72.75) (width 0.8) (layer "B.Cu") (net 6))
 (segment (start 106 72.75) (end 106 70.75) (width 0.8) (layer "B.Cu") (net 6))
 (segment (start 109.25 77) (end 109.25 75.25) (width 0.8) (layer "B.Cu") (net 6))
 (segment (start 109 75) (end 108.25 75) (width 0.8) (layer "B.Cu") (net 6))
 (segment (start 69.795 104.545) (end 73.8 104.545) (width 0.8) (layer "B.Cu") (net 20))
 (segment (start 64.5 102.225) (end 67.475 102.225) (width 0.8) (layer "B.Cu") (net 20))
 (segment (start 67.475 102.225) (end 69.795 104.545) (width 0.8) (layer "B.Cu") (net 20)))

